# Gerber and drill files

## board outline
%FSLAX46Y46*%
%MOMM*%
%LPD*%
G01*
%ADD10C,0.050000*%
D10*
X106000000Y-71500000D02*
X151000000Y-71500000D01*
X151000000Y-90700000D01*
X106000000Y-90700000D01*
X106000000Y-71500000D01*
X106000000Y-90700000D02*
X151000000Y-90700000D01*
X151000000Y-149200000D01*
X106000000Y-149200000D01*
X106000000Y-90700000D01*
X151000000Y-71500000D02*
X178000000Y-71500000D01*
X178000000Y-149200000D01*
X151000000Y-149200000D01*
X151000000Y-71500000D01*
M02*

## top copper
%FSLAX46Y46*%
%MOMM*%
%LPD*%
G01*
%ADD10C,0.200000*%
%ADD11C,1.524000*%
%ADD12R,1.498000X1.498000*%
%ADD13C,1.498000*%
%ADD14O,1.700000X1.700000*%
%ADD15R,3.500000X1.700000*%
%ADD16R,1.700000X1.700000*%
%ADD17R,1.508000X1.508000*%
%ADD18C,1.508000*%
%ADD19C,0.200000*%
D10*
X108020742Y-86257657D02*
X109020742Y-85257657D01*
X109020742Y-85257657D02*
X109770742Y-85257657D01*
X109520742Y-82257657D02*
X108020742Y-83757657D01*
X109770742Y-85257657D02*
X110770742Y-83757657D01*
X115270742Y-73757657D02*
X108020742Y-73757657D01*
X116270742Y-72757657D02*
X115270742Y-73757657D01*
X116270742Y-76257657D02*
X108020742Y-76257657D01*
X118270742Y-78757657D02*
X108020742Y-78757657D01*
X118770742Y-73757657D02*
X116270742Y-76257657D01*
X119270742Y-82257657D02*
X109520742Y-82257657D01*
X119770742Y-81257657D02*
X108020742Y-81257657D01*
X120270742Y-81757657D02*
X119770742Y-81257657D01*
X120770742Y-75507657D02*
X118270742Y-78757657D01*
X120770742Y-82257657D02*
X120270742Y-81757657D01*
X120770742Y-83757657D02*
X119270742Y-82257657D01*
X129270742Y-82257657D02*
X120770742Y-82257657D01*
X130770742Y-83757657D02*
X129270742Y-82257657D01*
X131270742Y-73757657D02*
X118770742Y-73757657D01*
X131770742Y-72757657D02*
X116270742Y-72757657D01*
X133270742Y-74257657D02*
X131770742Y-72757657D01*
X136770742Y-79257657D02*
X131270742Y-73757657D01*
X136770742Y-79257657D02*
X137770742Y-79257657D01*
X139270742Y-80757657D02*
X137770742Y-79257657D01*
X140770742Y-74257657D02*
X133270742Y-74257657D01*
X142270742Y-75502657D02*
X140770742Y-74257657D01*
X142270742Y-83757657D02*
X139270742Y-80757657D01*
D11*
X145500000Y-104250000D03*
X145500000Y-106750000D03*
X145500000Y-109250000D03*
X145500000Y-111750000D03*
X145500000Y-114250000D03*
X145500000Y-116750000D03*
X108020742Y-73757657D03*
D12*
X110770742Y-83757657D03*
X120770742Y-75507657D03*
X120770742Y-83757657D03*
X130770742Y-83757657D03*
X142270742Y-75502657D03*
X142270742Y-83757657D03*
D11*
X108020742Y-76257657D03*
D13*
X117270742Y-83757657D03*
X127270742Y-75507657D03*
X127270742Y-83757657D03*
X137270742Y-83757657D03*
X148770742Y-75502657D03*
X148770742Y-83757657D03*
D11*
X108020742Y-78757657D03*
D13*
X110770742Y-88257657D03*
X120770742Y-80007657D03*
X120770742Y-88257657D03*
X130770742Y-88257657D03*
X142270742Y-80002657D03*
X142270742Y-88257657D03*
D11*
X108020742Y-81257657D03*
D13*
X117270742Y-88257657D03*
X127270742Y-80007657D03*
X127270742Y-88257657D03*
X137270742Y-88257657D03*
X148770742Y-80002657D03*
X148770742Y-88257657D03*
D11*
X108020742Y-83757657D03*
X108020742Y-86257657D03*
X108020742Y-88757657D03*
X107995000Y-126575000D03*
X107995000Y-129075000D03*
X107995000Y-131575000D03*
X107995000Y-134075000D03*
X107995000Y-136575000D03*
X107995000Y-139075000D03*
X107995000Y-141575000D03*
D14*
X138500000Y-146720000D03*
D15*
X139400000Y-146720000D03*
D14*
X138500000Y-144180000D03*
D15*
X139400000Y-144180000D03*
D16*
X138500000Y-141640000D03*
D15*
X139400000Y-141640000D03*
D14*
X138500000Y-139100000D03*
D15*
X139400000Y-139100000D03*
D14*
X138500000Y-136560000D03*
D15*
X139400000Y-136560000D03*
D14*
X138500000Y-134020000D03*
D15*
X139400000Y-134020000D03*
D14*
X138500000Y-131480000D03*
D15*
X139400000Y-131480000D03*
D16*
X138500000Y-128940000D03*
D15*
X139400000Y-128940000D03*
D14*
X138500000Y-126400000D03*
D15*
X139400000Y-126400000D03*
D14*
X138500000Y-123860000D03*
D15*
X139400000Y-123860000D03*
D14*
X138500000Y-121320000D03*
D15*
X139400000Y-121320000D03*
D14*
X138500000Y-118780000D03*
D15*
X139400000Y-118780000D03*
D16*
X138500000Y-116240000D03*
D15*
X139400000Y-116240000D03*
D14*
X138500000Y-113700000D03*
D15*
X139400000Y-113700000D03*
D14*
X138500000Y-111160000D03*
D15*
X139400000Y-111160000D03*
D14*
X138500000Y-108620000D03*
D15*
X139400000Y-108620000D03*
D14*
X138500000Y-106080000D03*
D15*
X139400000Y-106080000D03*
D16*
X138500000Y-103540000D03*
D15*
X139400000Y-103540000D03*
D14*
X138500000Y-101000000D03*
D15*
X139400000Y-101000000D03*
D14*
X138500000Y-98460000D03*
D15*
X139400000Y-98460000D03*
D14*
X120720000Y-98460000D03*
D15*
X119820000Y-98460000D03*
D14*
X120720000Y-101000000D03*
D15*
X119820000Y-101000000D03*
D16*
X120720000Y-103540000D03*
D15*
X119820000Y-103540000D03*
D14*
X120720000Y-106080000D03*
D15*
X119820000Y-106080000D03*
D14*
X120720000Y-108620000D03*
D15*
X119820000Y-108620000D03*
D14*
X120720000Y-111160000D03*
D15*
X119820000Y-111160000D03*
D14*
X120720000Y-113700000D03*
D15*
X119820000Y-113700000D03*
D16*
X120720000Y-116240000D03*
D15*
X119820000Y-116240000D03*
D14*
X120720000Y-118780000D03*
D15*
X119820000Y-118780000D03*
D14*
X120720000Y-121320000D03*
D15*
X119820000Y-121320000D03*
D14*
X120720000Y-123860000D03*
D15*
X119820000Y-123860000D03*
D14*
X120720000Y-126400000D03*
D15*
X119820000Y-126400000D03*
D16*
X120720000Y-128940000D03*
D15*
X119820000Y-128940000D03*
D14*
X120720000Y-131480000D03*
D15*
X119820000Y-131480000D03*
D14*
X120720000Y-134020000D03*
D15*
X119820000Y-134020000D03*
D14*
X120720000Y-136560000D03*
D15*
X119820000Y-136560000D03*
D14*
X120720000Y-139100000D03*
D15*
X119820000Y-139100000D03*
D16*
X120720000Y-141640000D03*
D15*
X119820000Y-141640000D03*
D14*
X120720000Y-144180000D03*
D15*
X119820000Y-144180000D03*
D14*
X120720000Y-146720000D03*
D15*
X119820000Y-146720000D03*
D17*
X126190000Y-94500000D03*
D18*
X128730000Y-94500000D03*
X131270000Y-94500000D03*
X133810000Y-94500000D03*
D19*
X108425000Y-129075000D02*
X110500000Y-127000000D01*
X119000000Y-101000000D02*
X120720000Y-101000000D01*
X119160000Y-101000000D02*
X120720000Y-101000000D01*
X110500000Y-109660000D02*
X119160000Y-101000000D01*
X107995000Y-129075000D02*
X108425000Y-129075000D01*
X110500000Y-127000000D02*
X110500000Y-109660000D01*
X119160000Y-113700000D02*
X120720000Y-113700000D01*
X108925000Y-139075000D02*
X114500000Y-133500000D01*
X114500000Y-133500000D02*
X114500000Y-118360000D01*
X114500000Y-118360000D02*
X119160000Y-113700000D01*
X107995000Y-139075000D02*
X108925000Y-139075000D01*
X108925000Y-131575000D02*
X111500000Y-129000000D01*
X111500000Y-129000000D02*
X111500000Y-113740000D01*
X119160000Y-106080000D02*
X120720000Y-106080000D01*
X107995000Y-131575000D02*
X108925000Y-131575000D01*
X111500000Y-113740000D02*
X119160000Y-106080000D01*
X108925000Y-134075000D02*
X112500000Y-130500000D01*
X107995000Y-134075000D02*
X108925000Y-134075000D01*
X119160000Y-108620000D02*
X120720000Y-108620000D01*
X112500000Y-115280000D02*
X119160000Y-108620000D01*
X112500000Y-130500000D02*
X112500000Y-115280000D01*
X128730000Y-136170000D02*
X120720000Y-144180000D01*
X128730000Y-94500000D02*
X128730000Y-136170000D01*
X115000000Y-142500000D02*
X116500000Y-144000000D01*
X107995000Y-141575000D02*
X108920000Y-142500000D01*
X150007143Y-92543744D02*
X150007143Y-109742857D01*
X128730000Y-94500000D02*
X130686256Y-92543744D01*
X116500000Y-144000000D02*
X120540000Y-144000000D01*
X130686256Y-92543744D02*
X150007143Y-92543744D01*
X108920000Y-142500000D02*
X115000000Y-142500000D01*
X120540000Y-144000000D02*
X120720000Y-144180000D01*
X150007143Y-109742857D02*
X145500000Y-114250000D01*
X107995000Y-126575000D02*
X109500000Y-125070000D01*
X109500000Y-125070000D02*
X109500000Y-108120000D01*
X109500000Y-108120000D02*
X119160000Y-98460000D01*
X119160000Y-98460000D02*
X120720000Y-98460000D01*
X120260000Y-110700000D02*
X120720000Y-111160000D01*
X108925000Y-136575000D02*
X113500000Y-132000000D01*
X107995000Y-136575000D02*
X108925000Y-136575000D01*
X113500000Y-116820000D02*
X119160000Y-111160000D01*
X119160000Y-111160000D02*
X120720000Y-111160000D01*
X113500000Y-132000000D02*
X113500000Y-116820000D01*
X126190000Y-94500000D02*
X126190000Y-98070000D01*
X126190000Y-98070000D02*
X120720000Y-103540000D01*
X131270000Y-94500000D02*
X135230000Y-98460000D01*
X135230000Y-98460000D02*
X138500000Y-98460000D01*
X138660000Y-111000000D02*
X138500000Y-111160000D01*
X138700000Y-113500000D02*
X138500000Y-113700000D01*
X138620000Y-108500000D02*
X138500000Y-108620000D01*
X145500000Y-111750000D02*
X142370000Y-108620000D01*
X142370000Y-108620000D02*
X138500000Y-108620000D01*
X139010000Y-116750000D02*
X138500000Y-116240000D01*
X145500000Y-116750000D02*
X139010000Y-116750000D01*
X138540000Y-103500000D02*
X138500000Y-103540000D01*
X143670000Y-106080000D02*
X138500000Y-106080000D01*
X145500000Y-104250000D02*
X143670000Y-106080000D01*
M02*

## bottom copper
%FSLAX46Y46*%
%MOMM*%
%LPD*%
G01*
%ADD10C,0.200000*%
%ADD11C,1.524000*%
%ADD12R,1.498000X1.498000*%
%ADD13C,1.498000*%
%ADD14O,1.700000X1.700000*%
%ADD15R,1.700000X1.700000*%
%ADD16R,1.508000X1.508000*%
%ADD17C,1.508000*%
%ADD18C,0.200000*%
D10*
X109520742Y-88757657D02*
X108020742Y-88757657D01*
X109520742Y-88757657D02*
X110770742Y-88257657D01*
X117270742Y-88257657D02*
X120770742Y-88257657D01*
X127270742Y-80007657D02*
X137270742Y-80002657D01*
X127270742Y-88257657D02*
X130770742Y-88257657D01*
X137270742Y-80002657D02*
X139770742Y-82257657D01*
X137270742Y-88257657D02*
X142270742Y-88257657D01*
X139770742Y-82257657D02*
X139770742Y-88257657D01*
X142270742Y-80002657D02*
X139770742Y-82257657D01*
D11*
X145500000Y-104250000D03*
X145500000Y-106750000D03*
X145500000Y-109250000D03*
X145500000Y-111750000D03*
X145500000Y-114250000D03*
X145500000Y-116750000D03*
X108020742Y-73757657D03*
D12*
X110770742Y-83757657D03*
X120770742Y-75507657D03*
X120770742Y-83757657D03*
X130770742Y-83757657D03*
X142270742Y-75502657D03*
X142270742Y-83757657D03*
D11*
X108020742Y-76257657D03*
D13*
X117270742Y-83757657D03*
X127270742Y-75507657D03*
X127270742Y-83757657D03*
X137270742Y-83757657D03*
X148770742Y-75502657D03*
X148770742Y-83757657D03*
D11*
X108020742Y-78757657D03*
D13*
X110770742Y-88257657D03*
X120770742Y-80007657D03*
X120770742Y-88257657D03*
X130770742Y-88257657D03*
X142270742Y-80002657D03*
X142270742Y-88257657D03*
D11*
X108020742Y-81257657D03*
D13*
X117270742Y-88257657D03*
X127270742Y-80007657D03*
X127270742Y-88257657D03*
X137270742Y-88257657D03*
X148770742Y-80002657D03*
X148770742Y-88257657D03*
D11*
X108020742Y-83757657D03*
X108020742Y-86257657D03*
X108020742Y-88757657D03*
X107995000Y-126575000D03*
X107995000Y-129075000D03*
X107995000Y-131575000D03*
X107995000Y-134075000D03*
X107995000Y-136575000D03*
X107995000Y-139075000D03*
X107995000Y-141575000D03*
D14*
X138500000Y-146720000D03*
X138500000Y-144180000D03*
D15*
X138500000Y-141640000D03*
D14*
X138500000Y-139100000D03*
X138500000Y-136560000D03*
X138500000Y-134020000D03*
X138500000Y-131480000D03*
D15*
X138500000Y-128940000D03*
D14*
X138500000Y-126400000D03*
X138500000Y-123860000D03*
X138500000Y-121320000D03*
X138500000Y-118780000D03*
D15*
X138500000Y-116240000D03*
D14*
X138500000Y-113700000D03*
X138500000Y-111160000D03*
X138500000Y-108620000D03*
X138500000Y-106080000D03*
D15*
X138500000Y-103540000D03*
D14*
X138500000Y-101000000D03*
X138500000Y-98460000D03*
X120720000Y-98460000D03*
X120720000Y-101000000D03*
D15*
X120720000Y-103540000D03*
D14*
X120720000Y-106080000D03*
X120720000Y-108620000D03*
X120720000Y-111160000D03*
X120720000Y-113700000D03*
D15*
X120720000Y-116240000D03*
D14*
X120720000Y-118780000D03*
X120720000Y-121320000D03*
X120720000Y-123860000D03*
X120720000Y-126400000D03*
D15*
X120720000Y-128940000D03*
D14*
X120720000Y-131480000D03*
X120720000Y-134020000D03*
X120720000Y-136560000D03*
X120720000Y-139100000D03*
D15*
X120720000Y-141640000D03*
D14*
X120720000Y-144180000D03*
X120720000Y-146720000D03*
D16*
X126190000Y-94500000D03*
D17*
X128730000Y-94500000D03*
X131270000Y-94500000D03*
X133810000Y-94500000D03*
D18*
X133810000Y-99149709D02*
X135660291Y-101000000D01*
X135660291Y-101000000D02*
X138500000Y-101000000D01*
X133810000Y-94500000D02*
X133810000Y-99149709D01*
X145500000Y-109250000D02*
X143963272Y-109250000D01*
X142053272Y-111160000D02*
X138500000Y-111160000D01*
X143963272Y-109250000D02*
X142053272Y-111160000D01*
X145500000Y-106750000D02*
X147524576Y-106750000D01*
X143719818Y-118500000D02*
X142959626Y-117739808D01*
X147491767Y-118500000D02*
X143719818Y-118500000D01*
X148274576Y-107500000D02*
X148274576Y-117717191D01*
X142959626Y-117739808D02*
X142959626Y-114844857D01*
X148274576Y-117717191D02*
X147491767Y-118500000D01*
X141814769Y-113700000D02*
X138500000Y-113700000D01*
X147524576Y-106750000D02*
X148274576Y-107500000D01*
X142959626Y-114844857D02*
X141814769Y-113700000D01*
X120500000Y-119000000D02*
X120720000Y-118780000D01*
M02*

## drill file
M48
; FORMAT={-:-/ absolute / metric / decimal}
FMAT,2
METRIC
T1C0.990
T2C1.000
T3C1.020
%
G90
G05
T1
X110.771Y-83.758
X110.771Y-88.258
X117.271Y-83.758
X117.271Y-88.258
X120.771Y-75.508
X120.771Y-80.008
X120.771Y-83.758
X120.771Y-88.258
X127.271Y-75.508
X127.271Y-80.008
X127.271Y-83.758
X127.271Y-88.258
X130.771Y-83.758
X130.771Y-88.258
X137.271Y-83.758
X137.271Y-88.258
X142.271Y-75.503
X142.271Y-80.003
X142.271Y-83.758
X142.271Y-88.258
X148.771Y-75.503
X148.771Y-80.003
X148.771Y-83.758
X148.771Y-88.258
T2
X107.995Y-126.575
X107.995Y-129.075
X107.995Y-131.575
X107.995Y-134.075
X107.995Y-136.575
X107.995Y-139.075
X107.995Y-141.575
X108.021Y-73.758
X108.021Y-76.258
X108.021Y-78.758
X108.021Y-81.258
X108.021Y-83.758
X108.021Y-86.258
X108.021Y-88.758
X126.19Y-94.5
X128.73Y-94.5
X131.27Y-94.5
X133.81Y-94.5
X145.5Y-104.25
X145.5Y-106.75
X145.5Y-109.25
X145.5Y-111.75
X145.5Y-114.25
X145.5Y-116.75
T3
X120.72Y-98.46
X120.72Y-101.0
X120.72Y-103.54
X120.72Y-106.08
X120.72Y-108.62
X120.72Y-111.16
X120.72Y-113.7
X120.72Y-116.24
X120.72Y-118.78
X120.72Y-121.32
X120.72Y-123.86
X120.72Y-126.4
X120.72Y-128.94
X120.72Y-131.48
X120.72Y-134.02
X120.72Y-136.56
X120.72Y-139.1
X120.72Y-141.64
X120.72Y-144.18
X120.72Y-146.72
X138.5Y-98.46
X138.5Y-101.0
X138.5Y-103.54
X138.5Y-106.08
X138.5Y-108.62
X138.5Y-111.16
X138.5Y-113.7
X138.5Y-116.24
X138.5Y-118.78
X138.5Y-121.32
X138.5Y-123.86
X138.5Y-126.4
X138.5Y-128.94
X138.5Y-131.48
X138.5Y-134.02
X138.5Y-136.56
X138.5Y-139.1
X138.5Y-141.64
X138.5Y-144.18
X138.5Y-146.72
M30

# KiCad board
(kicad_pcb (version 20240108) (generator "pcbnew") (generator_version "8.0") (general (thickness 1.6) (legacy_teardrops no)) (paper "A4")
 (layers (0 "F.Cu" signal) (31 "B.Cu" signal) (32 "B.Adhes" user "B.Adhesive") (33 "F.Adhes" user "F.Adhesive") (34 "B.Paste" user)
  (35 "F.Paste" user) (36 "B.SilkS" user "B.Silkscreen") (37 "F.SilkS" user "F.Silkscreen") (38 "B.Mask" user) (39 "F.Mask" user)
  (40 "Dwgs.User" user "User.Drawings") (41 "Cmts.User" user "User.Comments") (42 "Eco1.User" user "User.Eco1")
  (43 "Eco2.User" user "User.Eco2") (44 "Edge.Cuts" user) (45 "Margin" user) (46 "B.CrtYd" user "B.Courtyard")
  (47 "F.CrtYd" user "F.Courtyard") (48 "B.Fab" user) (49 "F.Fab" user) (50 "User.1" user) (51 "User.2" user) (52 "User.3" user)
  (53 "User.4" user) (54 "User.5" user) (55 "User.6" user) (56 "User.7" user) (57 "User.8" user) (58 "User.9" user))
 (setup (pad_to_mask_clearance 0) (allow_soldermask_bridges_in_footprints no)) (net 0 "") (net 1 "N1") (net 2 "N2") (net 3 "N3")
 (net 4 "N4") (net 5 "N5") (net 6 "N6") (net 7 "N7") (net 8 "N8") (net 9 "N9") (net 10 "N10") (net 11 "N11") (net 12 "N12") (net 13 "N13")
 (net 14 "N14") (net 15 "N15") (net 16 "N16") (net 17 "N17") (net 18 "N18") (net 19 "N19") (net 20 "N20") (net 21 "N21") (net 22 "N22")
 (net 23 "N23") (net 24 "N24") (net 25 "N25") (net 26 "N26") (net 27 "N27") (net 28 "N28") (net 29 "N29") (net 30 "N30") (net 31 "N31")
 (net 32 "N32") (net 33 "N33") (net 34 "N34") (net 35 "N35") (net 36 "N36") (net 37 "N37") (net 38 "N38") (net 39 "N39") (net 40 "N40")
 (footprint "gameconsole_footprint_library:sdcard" (layer "F.Cu") (at 148.75 98.5 -90)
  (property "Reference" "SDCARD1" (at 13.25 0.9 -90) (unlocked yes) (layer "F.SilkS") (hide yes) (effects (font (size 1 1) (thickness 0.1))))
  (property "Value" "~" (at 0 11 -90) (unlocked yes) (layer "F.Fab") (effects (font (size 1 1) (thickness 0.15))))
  (pad "1" thru_hole circle (at 5.75 3.25 270) (size 1.524 1.524) (drill 1) (layers "*.Cu" "*.Mask") (remove_unused_layers no) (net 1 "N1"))
  (pad "2" thru_hole circle (at 8.25 3.25 270) (size 1.524 1.524) (drill 1) (layers "*.Cu" "*.Mask") (remove_unused_layers no) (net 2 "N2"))
  (pad "3" thru_hole circle (at 10.75 3.25 270) (size 1.524 1.524) (drill 1) (layers "*.Cu" "*.Mask") (remove_unused_layers no) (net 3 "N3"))
  (pad "4" thru_hole circle (at 13.25 3.25 270) (size 1.524 1.524) (drill 1) (layers "*.Cu" "*.Mask") (remove_unused_layers no) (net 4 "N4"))
  (pad "5" thru_hole circle (at 15.75 3.25 270) (size 1.524 1.524) (drill 1) (layers "*.Cu" "*.Mask") (remove_unused_layers no) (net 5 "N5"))
  (pad "6" thru_hole circle (at 18.25 3.25 270) (size 1.524 1.524) (drill 1) (layers "*.Cu" "*.Mask") (remove_unused_layers no) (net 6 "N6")))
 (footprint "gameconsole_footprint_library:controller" (layer "F.Cu") (at 106.525742 72.257657)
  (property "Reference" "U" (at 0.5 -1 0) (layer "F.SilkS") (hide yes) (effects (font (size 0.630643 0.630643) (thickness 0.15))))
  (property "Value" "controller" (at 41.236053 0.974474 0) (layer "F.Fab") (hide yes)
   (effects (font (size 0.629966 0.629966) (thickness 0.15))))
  (fp_line (start 1.495 14) (end 2.495 13) (stroke (width 0.2) (type default)) (layer "F.Cu"))
  (fp_line (start 2.495 13) (end 3.245 13) (stroke (width 0.2) (type default)) (layer "F.Cu"))
  (fp_line (start 2.995 10) (end 1.495 11.5) (stroke (width 0.2) (type default)) (layer "F.Cu"))
  (fp_line (start 3.245 13) (end 4.245 11.5) (stroke (width 0.2) (type default)) (layer "F.Cu"))
  (fp_line (start 8.745 1.5) (end 1.495 1.5) (stroke (width 0.2) (type default)) (layer "F.Cu"))
  (fp_line (start 9.745 0.5) (end 8.745 1.5) (stroke (width 0.2) (type default)) (layer "F.Cu"))
  (fp_line (start 9.745 4) (end 1.495 4) (stroke (width 0.2) (type default)) (layer "F.Cu"))
  (fp_line (start 11.745 6.5) (end 1.495 6.5) (stroke (width 0.2) (type default)) (layer "F.Cu"))
  (fp_line (start 12.245 1.5) (end 9.745 4) (stroke (width 0.2) (type default)) (layer "F.Cu"))
  (fp_line (start 12.745 10) (end 2.995 10) (stroke (width 0.2) (type default)) (layer "F.Cu"))
  (fp_line (start 13.245 9) (end 1.495 9) (stroke (width 0.2) (type default)) (layer "F.Cu"))
  (fp_line (start 13.745 9.5) (end 13.245 9) (stroke (width 0.2) (type default)) (layer "F.Cu"))
  (fp_line (start 14.245 3.25) (end 11.745 6.5) (stroke (width 0.2) (type default)) (layer "F.Cu"))
  (fp_line (start 14.245 10) (end 13.745 9.5) (stroke (width 0.2) (type default)) (layer "F.Cu"))
  (fp_line (start 14.245 11.5) (end 12.745 10) (stroke (width 0.2) (type default)) (layer "F.Cu"))
  (fp_line (start 22.745 10) (end 14.245 10) (stroke (width 0.2) (type default)) (layer "F.Cu"))
  (fp_line (start 24.245 11.5) (end 22.745 10) (stroke (width 0.2) (type default)) (layer "F.Cu"))
  (fp_line (start 24.745 1.5) (end 12.245 1.5) (stroke (width 0.2) (type default)) (layer "F.Cu"))
  (fp_line (start 25.245 0.5) (end 9.745 0.5) (stroke (width 0.2) (type default)) (layer "F.Cu"))
  (fp_line (start 26.745 2) (end 25.245 0.5) (stroke (width 0.2) (type default)) (layer "F.Cu"))
  (fp_line (start 30.245 7) (end 24.745 1.5) (stroke (width 0.2) (type default)) (layer "F.Cu"))
  (fp_line (start 30.245 7) (end 31.245 7) (stroke (width 0.2) (type default)) (layer "F.Cu"))
  (fp_line (start 32.745 8.5) (end 31.245 7) (stroke (width 0.2) (type default)) (layer "F.Cu"))
  (fp_line (start 34.245 2) (end 26.745 2) (stroke (width 0.2) (type default)) (layer "F.Cu"))
  (fp_line (start 35.745 3.245) (end 34.245 2) (stroke (width 0.2) (type default)) (layer "F.Cu"))
  (fp_line (start 35.745 11.5) (end 32.745 8.5) (stroke (width 0.2) (type default)) (layer "F.Cu"))
  (fp_line (start 2.995 16.5) (end 1.495 16.5) (stroke (width 0.2) (type default)) (layer "B.Cu"))
  (fp_line (start 2.995 16.5) (end 4.245 16) (stroke (width 0.2) (type default)) (layer "B.Cu"))
  (fp_line (start 10.745 16) (end 14.245 16) (stroke (width 0.2) (type default)) (layer "B.Cu"))
  (fp_line (start 20.745 7.75) (end 30.745 7.745) (stroke (width 0.2) (type default)) (layer "B.Cu"))
  (fp_line (start 20.745 16) (end 24.245 16) (stroke (width 0.2) (type default)) (layer "B.Cu"))
  (fp_line (start 30.745 7.745) (end 33.245 10) (stroke (width 0.2) (type default)) (layer "B.Cu"))
  (fp_line (start 30.745 16) (end 35.745 16) (stroke (width 0.2) (type default)) (layer "B.Cu"))
  (fp_line (start 33.245 10) (end 33.245 16) (stroke (width 0.2) (type default)) (layer "B.Cu"))
  (fp_line (start 35.745 7.745) (end 33.245 10) (stroke (width 0.2) (type default)) (layer "B.Cu"))
  (pad "1" thru_hole circle (at 1.495 1.5) (size 1.524 1.524) (drill 1) (layers "*.Cu" "*.Mask") (remove_unused_layers no))
  (pad "1" thru_hole rect (at 4.245 11.5) (size 1.498 1.498) (drill 0.99) (layers "*.Cu" "*.Mask") (remove_unused_layers no)
   (solder_mask_margin 0.102))
  (pad "1" thru_hole rect (at 14.245 3.25) (size 1.498 1.498) (drill 0.99) (layers "*.Cu" "*.Mask") (remove_unused_layers no)
   (solder_mask_margin 0.102))
  (pad "1" thru_hole rect (at 14.245 11.5) (size 1.498 1.498) (drill 0.99) (layers "*.Cu" "*.Mask") (remove_unused_layers no)
   (solder_mask_margin 0.102))
  (pad "1" thru_hole rect (at 24.245 11.5) (size 1.498 1.498) (drill 0.99) (layers "*.Cu" "*.Mask") (remove_unused_layers no)
   (solder_mask_margin 0.102))
  (pad "1" thru_hole rect (at 35.745 3.245) (size 1.498 1.498) (drill 0.99) (layers "*.Cu" "*.Mask") (remove_unused_layers no)
   (solder_mask_margin 0.102))
  (pad "1" thru_hole rect (at 35.745 11.5) (size 1.498 1.498) (drill 0.99) (layers "*.Cu" "*.Mask") (remove_unused_layers no)
   (solder_mask_margin 0.102))
  (pad "2" thru_hole circle (at 1.495 4) (size 1.524 1.524) (drill 1) (layers "*.Cu" "*.Mask") (remove_unused_layers no))
  (pad "2" thru_hole circle (at 10.745 11.5) (size 1.498 1.498) (drill 0.99) (layers "*.Cu" "*.Mask") (remove_unused_layers no)
   (solder_mask_margin 0.102))
  (pad "2" thru_hole circle (at 20.745 3.25) (size 1.498 1.498) (drill 0.99) (layers "*.Cu" "*.Mask") (remove_unused_layers no)
   (solder_mask_margin 0.102))
  (pad "2" thru_hole circle (at 20.745 11.5) (size 1.498 1.498) (drill 0.99) (layers "*.Cu" "*.Mask") (remove_unused_layers no)
   (solder_mask_margin 0.102))
  (pad "2" thru_hole circle (at 30.745 11.5) (size 1.498 1.498) (drill 0.99) (layers "*.Cu" "*.Mask") (remove_unused_layers no)
   (solder_mask_margin 0.102))
  (pad "2" thru_hole circle (at 42.245 3.245) (size 1.498 1.498) (drill 0.99) (layers "*.Cu" "*.Mask") (remove_unused_layers no)
   (solder_mask_margin 0.102))
  (pad "2" thru_hole circle (at 42.245 11.5) (size 1.498 1.498) (drill 0.99) (layers "*.Cu" "*.Mask") (remove_unused_layers no)
   (solder_mask_margin 0.102))
  (pad "3" thru_hole circle (at 1.495 6.5) (size 1.524 1.524) (drill 1) (layers "*.Cu" "*.Mask") (remove_unused_layers no))
  (pad "3" thru_hole circle (at 4.245 16) (size 1.498 1.498) (drill 0.99) (layers "*.Cu" "*.Mask") (remove_unused_layers no)
   (solder_mask_margin 0.102))
  (pad "3" thru_hole circle (at 14.245 7.75) (size 1.498 1.498) (drill 0.99) (layers "*.Cu" "*.Mask") (remove_unused_layers no)
   (solder_mask_margin 0.102))
  (pad "3" thru_hole circle (at 14.245 16) (size 1.498 1.498) (drill 0.99) (layers "*.Cu" "*.Mask") (remove_unused_layers no)
   (solder_mask_margin 0.102))
  (pad "3" thru_hole circle (at 24.245 16) (size 1.498 1.498) (drill 0.99) (layers "*.Cu" "*.Mask") (remove_unused_layers no)
   (solder_mask_margin 0.102))
  (pad "3" thru_hole circle (at 35.745 7.745) (size 1.498 1.498) (drill 0.99) (layers "*.Cu" "*.Mask") (remove_unused_layers no)
   (solder_mask_margin 0.102))
  (pad "3" thru_hole circle (at 35.745 16) (size 1.498 1.498) (drill 0.99) (layers "*.Cu" "*.Mask") (remove_unused_layers no)
   (solder_mask_margin 0.102))
  (pad "4" thru_hole circle (at 1.495 9) (size 1.524 1.524) (drill 1) (layers "*.Cu" "*.Mask") (remove_unused_layers no))
  (pad "4" thru_hole circle (at 10.745 16) (size 1.498 1.498) (drill 0.99) (layers "*.Cu" "*.Mask") (remove_unused_layers no)
   (solder_mask_margin 0.102))
  (pad "4" thru_hole circle (at 20.745 7.75) (size 1.498 1.498) (drill 0.99) (layers "*.Cu" "*.Mask") (remove_unused_layers no)
   (solder_mask_margin 0.102))
  (pad "4" thru_hole circle (at 20.745 16) (size 1.498 1.498) (drill 0.99) (layers "*.Cu" "*.Mask") (remove_unused_layers no)
   (solder_mask_margin 0.102))
  (pad "4" thru_hole circle (at 30.745 16) (size 1.498 1.498) (drill 0.99) (layers "*.Cu" "*.Mask") (remove_unused_layers no)
   (solder_mask_margin 0.102))
  (pad "4" thru_hole circle (at 42.245 7.745) (size 1.498 1.498) (drill 0.99) (layers "*.Cu" "*.Mask") (remove_unused_layers no)
   (solder_mask_margin 0.102))
  (pad "4" thru_hole circle (at 42.245 16) (size 1.498 1.498) (drill 0.99) (layers "*.Cu" "*.Mask") (remove_unused_layers no)
   (solder_mask_margin 0.102))
  (pad "5" thru_hole circle (at 1.495 11.5) (size 1.524 1.524) (drill 1) (layers "*.Cu" "*.Mask") (remove_unused_layers no))
  (pad "6" thru_hole circle (at 1.495 14) (size 1.524 1.524) (drill 1) (layers "*.Cu" "*.Mask") (remove_unused_layers no))
  (pad "7" thru_hole circle (at 1.495 16.5) (size 1.524 1.524) (drill 1) (layers "*.Cu" "*.Mask") (remove_unused_layers no)))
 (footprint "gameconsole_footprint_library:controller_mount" (layer "F.Cu") (at 106.5 125.075)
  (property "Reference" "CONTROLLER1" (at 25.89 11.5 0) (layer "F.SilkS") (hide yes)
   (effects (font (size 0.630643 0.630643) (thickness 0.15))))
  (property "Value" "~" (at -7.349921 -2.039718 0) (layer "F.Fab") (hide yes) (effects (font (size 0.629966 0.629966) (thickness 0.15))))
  (pad "1" thru_hole circle (at 1.495 1.5) (size 1.524 1.524) (drill 1) (layers "*.Cu" "*.Mask") (remove_unused_layers no) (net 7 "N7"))
  (pad "2" thru_hole circle (at 1.495 4) (size 1.524 1.524) (drill 1) (layers "*.Cu" "*.Mask") (remove_unused_layers no) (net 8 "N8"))
  (pad "3" thru_hole circle (at 1.495 6.5) (size 1.524 1.524) (drill 1) (layers "*.Cu" "*.Mask") (remove_unused_layers no) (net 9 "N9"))
  (pad "4" thru_hole circle (at 1.495 9) (size 1.524 1.524) (drill 1) (layers "*.Cu" "*.Mask") (remove_unused_layers no) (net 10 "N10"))
  (pad "5" thru_hole circle (at 1.495 11.5) (size 1.524 1.524) (drill 1) (layers "*.Cu" "*.Mask") (remove_unused_layers no) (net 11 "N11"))
  (pad "6" thru_hole circle (at 1.495 14) (size 1.524 1.524) (drill 1) (layers "*.Cu" "*.Mask") (remove_unused_layers no) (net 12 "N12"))
  (pad "7" thru_hole circle (at 1.495 16.5) (size 1.524 1.524) (drill 1) (layers "*.Cu" "*.Mask") (remove_unused_layers no) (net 5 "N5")))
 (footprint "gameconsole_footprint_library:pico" (layer "F.Cu") (at 129.61 122.59 180)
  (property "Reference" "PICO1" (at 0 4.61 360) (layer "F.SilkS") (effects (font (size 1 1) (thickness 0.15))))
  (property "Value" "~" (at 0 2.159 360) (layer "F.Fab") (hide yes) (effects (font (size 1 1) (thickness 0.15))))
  (pad "1" thru_hole oval (at -8.89 -24.13 180) (size 1.7 1.7) (drill 1.02) (layers "*.Cu" "*.Mask") (remove_unused_layers no)
   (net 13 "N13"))
  (pad "1" smd rect (at -8.89 -24.13 180) (size 3.5 1.7) (drill (offset -0.9 0)) (layers "F.Cu" "F.Mask") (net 13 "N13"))
  (pad "2" thru_hole oval (at -8.89 -21.59 180) (size 1.7 1.7) (drill 1.02) (layers "*.Cu" "*.Mask") (remove_unused_layers no)
   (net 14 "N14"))
  (pad "2" smd rect (at -8.89 -21.59 180) (size 3.5 1.7) (drill (offset -0.9 0)) (layers "F.Cu" "F.Mask") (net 14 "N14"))
  (pad "3" thru_hole rect (at -8.89 -19.05 180) (size 1.7 1.7) (drill 1.02) (layers "*.Cu" "*.Mask") (remove_unused_layers no)
   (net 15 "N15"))
  (pad "3" smd rect (at -8.89 -19.05 180) (size 3.5 1.7) (drill (offset -0.9 0)) (layers "F.Cu" "F.Mask") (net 15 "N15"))
  (pad "4" thru_hole oval (at -8.89 -16.51 180) (size 1.7 1.7) (drill 1.02) (layers "*.Cu" "*.Mask") (remove_unused_layers no)
   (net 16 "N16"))
  (pad "4" smd rect (at -8.89 -16.51 180) (size 3.5 1.7) (drill (offset -0.9 0)) (layers "F.Cu" "F.Mask") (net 16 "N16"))
  (pad "5" thru_hole oval (at -8.89 -13.97 180) (size 1.7 1.7) (drill 1.02) (layers "*.Cu" "*.Mask") (remove_unused_layers no)
   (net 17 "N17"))
  (pad "5" smd rect (at -8.89 -13.97 180) (size 3.5 1.7) (drill (offset -0.9 0)) (layers "F.Cu" "F.Mask") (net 17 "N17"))
  (pad "6" thru_hole oval (at -8.89 -11.43 180) (size 1.7 1.7) (drill 1.02) (layers "*.Cu" "*.Mask") (remove_unused_layers no)
   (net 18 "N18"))
  (pad "6" smd rect (at -8.89 -11.43 180) (size 3.5 1.7) (drill (offset -0.9 0)) (layers "F.Cu" "F.Mask") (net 18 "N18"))
  (pad "7" thru_hole oval (at -8.89 -8.89 180) (size 1.7 1.7) (drill 1.02) (layers "*.Cu" "*.Mask") (remove_unused_layers no) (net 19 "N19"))
  (pad "7" smd rect (at -8.89 -8.89 180) (size 3.5 1.7) (drill (offset -0.9 0)) (layers "F.Cu" "F.Mask") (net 19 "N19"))
  (pad "8" thru_hole rect (at -8.89 -6.35 180) (size 1.7 1.7) (drill 1.02) (layers "*.Cu" "*.Mask") (remove_unused_layers no) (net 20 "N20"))
  (pad "8" smd rect (at -8.89 -6.35 180) (size 3.5 1.7) (drill (offset -0.9 0)) (layers "F.Cu" "F.Mask") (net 20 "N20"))
  (pad "9" thru_hole oval (at -8.89 -3.81 180) (size 1.7 1.7) (drill 1.02) (layers "*.Cu" "*.Mask") (remove_unused_layers no) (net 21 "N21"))
  (pad "9" smd rect (at -8.89 -3.81 180) (size 3.5 1.7) (drill (offset -0.9 0)) (layers "F.Cu" "F.Mask") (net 21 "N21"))
  (pad "10" thru_hole oval (at -8.89 -1.27 180) (size 1.7 1.7) (drill 1.02) (layers "*.Cu" "*.Mask") (remove_unused_layers no)
   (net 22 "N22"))
  (pad "10" smd rect (at -8.89 -1.27 180) (size 3.5 1.7) (drill (offset -0.9 0)) (layers "F.Cu" "F.Mask") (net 22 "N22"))
  (pad "11" thru_hole oval (at -8.89 1.27 180) (size 1.7 1.7) (drill 1.02) (layers "*.Cu" "*.Mask") (remove_unused_layers no) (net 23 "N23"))
  (pad "11" smd rect (at -8.89 1.27 180) (size 3.5 1.7) (drill (offset -0.9 0)) (layers "F.Cu" "F.Mask") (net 23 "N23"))
  (pad "12" thru_hole oval (at -8.89 3.81 180) (size 1.7 1.7) (drill 1.02) (layers "*.Cu" "*.Mask") (remove_unused_layers no) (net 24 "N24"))
  (pad "12" smd rect (at -8.89 3.81 180) (size 3.5 1.7) (drill (offset -0.9 0)) (layers "F.Cu" "F.Mask") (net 24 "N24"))
  (pad "13" thru_hole rect (at -8.89 6.35 180) (size 1.7 1.7) (drill 1.02) (layers "*.Cu" "*.Mask") (remove_unused_layers no) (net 6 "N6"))
  (pad "13" smd rect (at -8.89 6.35 180) (size 3.5 1.7) (drill (offset -0.9 0)) (layers "F.Cu" "F.Mask") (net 6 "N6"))
  (pad "14" thru_hole oval (at -8.89 8.89 180) (size 1.7 1.7) (drill 1.02) (layers "*.Cu" "*.Mask") (remove_unused_layers no) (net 2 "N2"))
  (pad "14" smd rect (at -8.89 8.89 180) (size 3.5 1.7) (drill (offset -0.9 0)) (layers "F.Cu" "F.Mask") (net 2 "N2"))
  (pad "15" thru_hole oval (at -8.89 11.43 180) (size 1.7 1.7) (drill 1.02) (layers "*.Cu" "*.Mask") (remove_unused_layers no) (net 3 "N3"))
  (pad "15" smd rect (at -8.89 11.43 180) (size 3.5 1.7) (drill (offset -0.9 0)) (layers "F.Cu" "F.Mask") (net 3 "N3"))
  (pad "16" thru_hole oval (at -8.89 13.97 180) (size 1.7 1.7) (drill 1.02) (layers "*.Cu" "*.Mask") (remove_unused_layers no) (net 4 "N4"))
  (pad "16" smd rect (at -8.89 13.97 180) (size 3.5 1.7) (drill (offset -0.9 0)) (layers "F.Cu" "F.Mask") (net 4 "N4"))
  (pad "17" thru_hole oval (at -8.89 16.51 180) (size 1.7 1.7) (drill 1.02) (layers "*.Cu" "*.Mask") (remove_unused_layers no) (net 1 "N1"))
  (pad "17" smd rect (at -8.89 16.51 180) (size 3.5 1.7) (drill (offset -0.9 0)) (layers "F.Cu" "F.Mask") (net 1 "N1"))
  (pad "18" thru_hole rect (at -8.89 19.05 180) (size 1.7 1.7) (drill 1.02) (layers "*.Cu" "*.Mask") (remove_unused_layers no)
   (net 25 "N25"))
  (pad "18" smd rect (at -8.89 19.05 180) (size 3.5 1.7) (drill (offset -0.9 0)) (layers "F.Cu" "F.Mask") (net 25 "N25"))
  (pad "19" thru_hole oval (at -8.89 21.59 180) (size 1.7 1.7) (drill 1.02) (layers "*.Cu" "*.Mask") (remove_unused_layers no)
   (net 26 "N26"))
  (pad "19" smd rect (at -8.89 21.59 180) (size 3.5 1.7) (drill (offset -0.9 0)) (layers "F.Cu" "F.Mask") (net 26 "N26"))
  (pad "20" thru_hole oval (at -8.89 24.13 180) (size 1.7 1.7) (drill 1.02) (layers "*.Cu" "*.Mask") (remove_unused_layers no)
   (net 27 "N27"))
  (pad "20" smd rect (at -8.89 24.13 180) (size 3.5 1.7) (drill (offset -0.9 0)) (layers "F.Cu" "F.Mask") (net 27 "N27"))
  (pad "21" thru_hole oval (at 8.89 24.13 180) (size 1.7 1.7) (drill 1.02) (layers "*.Cu" "*.Mask") (remove_unused_layers no) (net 7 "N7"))
  (pad "21" smd rect (at 8.89 24.13 180) (size 3.5 1.7) (drill (offset 0.9 0)) (layers "F.Cu" "F.Mask") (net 7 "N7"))
  (pad "22" thru_hole oval (at 8.89 21.59 180) (size 1.7 1.7) (drill 1.02) (layers "*.Cu" "*.Mask") (remove_unused_layers no) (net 8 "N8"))
  (pad "22" smd rect (at 8.89 21.59 180) (size 3.5 1.7) (drill (offset 0.9 0)) (layers "F.Cu" "F.Mask") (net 8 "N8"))
  (pad "23" thru_hole rect (at 8.89 19.05 180) (size 1.7 1.7) (drill 1.02) (layers "*.Cu" "*.Mask") (remove_unused_layers no) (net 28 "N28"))
  (pad "23" smd rect (at 8.89 19.05 180) (size 3.5 1.7) (drill (offset 0.9 0)) (layers "F.Cu" "F.Mask") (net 28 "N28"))
  (pad "24" thru_hole oval (at 8.89 16.51 180) (size 1.7 1.7) (drill 1.02) (layers "*.Cu" "*.Mask") (remove_unused_layers no) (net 9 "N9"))
  (pad "24" smd rect (at 8.89 16.51 180) (size 3.5 1.7) (drill (offset 0.9 0)) (layers "F.Cu" "F.Mask") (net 9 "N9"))
  (pad "25" thru_hole oval (at 8.89 13.97 180) (size 1.7 1.7) (drill 1.02) (layers "*.Cu" "*.Mask") (remove_unused_layers no) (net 10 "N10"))
  (pad "25" smd rect (at 8.89 13.97 180) (size 3.5 1.7) (drill (offset 0.9 0)) (layers "F.Cu" "F.Mask") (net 10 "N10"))
  (pad "26" thru_hole oval (at 8.89 11.43 180) (size 1.7 1.7) (drill 1.02) (layers "*.Cu" "*.Mask") (remove_unused_layers no) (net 11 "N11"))
  (pad "26" smd rect (at 8.89 11.43 180) (size 3.5 1.7) (drill (offset 0.9 0)) (layers "F.Cu" "F.Mask") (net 11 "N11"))
  (pad "27" thru_hole oval (at 8.89 8.89 180) (size 1.7 1.7) (drill 1.02) (layers "*.Cu" "*.Mask") (remove_unused_layers no) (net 12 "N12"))
  (pad "27" smd rect (at 8.89 8.89 180) (size 3.5 1.7) (drill (offset 0.9 0)) (layers "F.Cu" "F.Mask") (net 12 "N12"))
  (pad "28" thru_hole rect (at 8.89 6.35 180) (size 1.7 1.7) (drill 1.02) (layers "*.Cu" "*.Mask") (remove_unused_layers no) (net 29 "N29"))
  (pad "28" smd rect (at 8.89 6.35 180) (size 3.5 1.7) (drill (offset 0.9 0)) (layers "F.Cu" "F.Mask") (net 29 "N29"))
  (pad "29" thru_hole oval (at 8.89 3.81 180) (size 1.7 1.7) (drill 1.02) (layers "*.Cu" "*.Mask") (remove_unused_layers no) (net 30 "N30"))
  (pad "29" smd rect (at 8.89 3.81 180) (size 3.5 1.7) (drill (offset 0.9 0)) (layers "F.Cu" "F.Mask") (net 30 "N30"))
  (pad "30" thru_hole oval (at 8.89 1.27 180) (size 1.7 1.7) (drill 1.02) (layers "*.Cu" "*.Mask") (remove_unused_layers no) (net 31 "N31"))
  (pad "30" smd rect (at 8.89 1.27 180) (size 3.5 1.7) (drill (offset 0.9 0)) (layers "F.Cu" "F.Mask") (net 31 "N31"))
  (pad "31" thru_hole oval (at 8.89 -1.27 180) (size 1.7 1.7) (drill 1.02) (layers "*.Cu" "*.Mask") (remove_unused_layers no) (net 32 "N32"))
  (pad "31" smd rect (at 8.89 -1.27 180) (size 3.5 1.7) (drill (offset 0.9 0)) (layers "F.Cu" "F.Mask") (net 32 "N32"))
  (pad "32" thru_hole oval (at 8.89 -3.81 180) (size 1.7 1.7) (drill 1.02) (layers "*.Cu" "*.Mask") (remove_unused_layers no) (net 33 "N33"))
  (pad "32" smd rect (at 8.89 -3.81 180) (size 3.5 1.7) (drill (offset 0.9 0)) (layers "F.Cu" "F.Mask") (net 33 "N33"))
  (pad "33" thru_hole rect (at 8.89 -6.35 180) (size 1.7 1.7) (drill 1.02) (layers "*.Cu" "*.Mask") (remove_unused_layers no) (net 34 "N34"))
  (pad "33" smd rect (at 8.89 -6.35 180) (size 3.5 1.7) (drill (offset 0.9 0)) (layers "F.Cu" "F.Mask") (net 34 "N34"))
  (pad "34" thru_hole oval (at 8.89 -8.89 180) (size 1.7 1.7) (drill 1.02) (layers "*.Cu" "*.Mask") (remove_unused_layers no) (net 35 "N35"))
  (pad "34" smd rect (at 8.89 -8.89 180) (size 3.5 1.7) (drill (offset 0.9 0)) (layers "F.Cu" "F.Mask") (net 35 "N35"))
  (pad "35" thru_hole oval (at 8.89 -11.43 180) (size 1.7 1.7) (drill 1.02) (layers "*.Cu" "*.Mask") (remove_unused_layers no)
   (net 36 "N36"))
  (pad "35" smd rect (at 8.89 -11.43 180) (size 3.5 1.7) (drill (offset 0.9 0)) (layers "F.Cu" "F.Mask") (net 36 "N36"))
  (pad "36" thru_hole oval (at 8.89 -13.97 180) (size 1.7 1.7) (drill 1.02) (layers "*.Cu" "*.Mask") (remove_unused_layers no)
   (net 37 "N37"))
  (pad "36" smd rect (at 8.89 -13.97 180) (size 3.5 1.7) (drill (offset 0.9 0)) (layers "F.Cu" "F.Mask") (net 37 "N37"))
  (pad "37" thru_hole oval (at 8.89 -16.51 180) (size 1.7 1.7) (drill 1.02) (layers "*.Cu" "*.Mask") (remove_unused_layers no)
   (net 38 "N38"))
  (pad "37" smd rect (at 8.89 -16.51 180) (size 3.5 1.7) (drill (offset 0.9 0)) (layers "F.Cu" "F.Mask") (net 38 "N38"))
  (pad "38" thru_hole rect (at 8.89 -19.05 180) (size 1.7 1.7) (drill 1.02) (layers "*.Cu" "*.Mask") (remove_unused_layers no)
   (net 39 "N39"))
  (pad "38" smd rect (at 8.89 -19.05 180) (size 3.5 1.7) (drill (offset 0.9 0)) (layers "F.Cu" "F.Mask") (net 39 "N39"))
  (pad "39" thru_hole oval (at 8.89 -21.59 180) (size 1.7 1.7) (drill 1.02) (layers "*.Cu" "*.Mask") (remove_unused_layers no) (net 5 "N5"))
  (pad "39" smd rect (at 8.89 -21.59 180) (size 3.5 1.7) (drill (offset 0.9 0)) (layers "F.Cu" "F.Mask") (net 5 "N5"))
  (pad "40" thru_hole oval (at 8.89 -24.13 180) (size 1.7 1.7) (drill 1.02) (layers "*.Cu" "*.Mask") (remove_unused_layers no)
   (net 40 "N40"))
  (pad "40" smd rect (at 8.89 -24.13 180) (size 3.5 1.7) (drill (offset 0.9 0)) (layers "F.Cu" "F.Mask") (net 40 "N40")))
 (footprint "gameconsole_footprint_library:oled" (layer "F.Cu") (at 130 106)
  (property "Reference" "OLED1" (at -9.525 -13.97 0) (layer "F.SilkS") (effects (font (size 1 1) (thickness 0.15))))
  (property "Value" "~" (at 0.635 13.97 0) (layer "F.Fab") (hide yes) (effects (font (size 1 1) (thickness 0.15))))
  (pad "1" thru_hole rect (at -3.81 -11.5) (size 1.508 1.508) (drill 1) (layers "*.Cu" "*.Mask") (remove_unused_layers no) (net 28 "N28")
   (solder_mask_margin 0.102))
  (pad "2" thru_hole circle (at -1.27 -11.5) (size 1.508 1.508) (drill 1) (layers "*.Cu" "*.Mask") (remove_unused_layers no) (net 5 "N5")
   (solder_mask_margin 0.102))
  (pad "3" thru_hole circle (at 1.27 -11.5) (size 1.508 1.508) (drill 1) (layers "*.Cu" "*.Mask") (remove_unused_layers no) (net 27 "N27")
   (solder_mask_margin 0.102))
  (pad "4" thru_hole circle (at 3.81 -11.5) (size 1.508 1.508) (drill 1) (layers "*.Cu" "*.Mask") (remove_unused_layers no) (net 26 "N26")
   (solder_mask_margin 0.102)))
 (gr_rect (start 106 71.5) (end 151 90.7) (stroke (width 0.05) (type default)) (fill none) (layer "Edge.Cuts"))
 (gr_rect (start 106 90.7) (end 151 149.2) (stroke (width 0.05) (type default)) (fill none) (layer "Edge.Cuts"))
 (gr_rect (start 151 71.5) (end 178 149.2) (stroke (width 0.05) (type default)) (fill none) (layer "Edge.Cuts"))
 (segment (start 108.425 129.075) (end 110.5 127) (width 0.2) (layer "F.Cu") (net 8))
 (segment (start 119 101) (end 120.72 101) (width 0.2) (layer "F.Cu") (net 8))
 (segment (start 119.16 101) (end 120.72 101) (width 0.2) (layer "F.Cu") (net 8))
 (segment (start 110.5 109.66) (end 119.16 101) (width 0.2) (layer "F.Cu") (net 8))
 (segment (start 107.995 129.075) (end 108.425 129.075) (width 0.2) (layer "F.Cu") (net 8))
 (segment (start 110.5 127) (end 110.5 109.66) (width 0.2) (layer "F.Cu") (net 8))
 (segment (start 119.16 113.7) (end 120.72 113.7) (width 0.2) (layer "F.Cu") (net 12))
 (segment (start 108.925 139.075) (end 114.5 133.5) (width 0.2) (layer "F.Cu") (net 12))
 (segment (start 114.5 133.5) (end 114.5 118.36) (width 0.2) (layer "F.Cu") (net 12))
 (segment (start 114.5 118.36) (end 119.16 113.7) (width 0.2) (layer "F.Cu") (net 12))
 (segment (start 107.995 139.075) (end 108.925 139.075) (width 0.2) (layer "F.Cu") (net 12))
 (segment (start 108.925 131.575) (end 111.5 129) (width 0.2) (layer "F.Cu") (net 9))
 (segment (start 111.5 129) (end 111.5 113.74) (width 0.2) (layer "F.Cu") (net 9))
 (segment (start 119.16 106.08) (end 120.72 106.08) (width 0.2) (layer "F.Cu") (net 9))
 (segment (start 107.995 131.575) (end 108.925 131.575) (width 0.2) (layer "F.Cu") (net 9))
 (segment (start 111.5 113.74) (end 119.16 106.08) (width 0.2) (layer "F.Cu") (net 9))
 (segment (start 108.925 134.075) (end 112.5 130.5) (width 0.2) (layer "F.Cu") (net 10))
 (segment (start 107.995 134.075) (end 108.925 134.075) (width 0.2) (layer "F.Cu") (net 10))
 (segment (start 119.16 108.62) (end 120.72 108.62) (width 0.2) (layer "F.Cu") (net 10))
 (segment (start 112.5 115.28) (end 119.16 108.62) (width 0.2) (layer "F.Cu") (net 10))
 (segment (start 112.5 130.5) (end 112.5 115.28) (width 0.2) (layer "F.Cu") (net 10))
 (segment (start 128.73 136.17) (end 120.72 144.18) (width 0.2) (layer "F.Cu") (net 5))
 (segment (start 128.73 94.5) (end 128.73 136.17) (width 0.2) (layer "F.Cu") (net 5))
 (segment (start 115 142.5) (end 116.5 144) (width 0.2) (layer "F.Cu") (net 5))
 (segment (start 107.995 141.575) (end 108.92 142.5) (width 0.2) (layer "F.Cu") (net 5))
 (segment (start 150.007143 92.543744) (end 150.007143 109.742857) (width 0.2) (layer "F.Cu") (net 5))
 (segment (start 128.73 94.5) (end 130.686256 92.543744) (width 0.2) (layer "F.Cu") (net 5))
 (segment (start 116.5 144) (end 120.54 144) (width 0.2) (layer "F.Cu") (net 5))
 (segment (start 130.686256 92.543744) (end 150.007143 92.543744) (width 0.2) (layer "F.Cu") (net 5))
 (segment (start 108.92 142.5) (end 115 142.5) (width 0.2) (layer "F.Cu") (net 5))
 (segment (start 120.54 144) (end 120.72 144.18) (width 0.2) (layer "F.Cu") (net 5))
 (segment (start 150.007143 109.742857) (end 145.5 114.25) (width 0.2) (layer "F.Cu") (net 5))
 (segment (start 107.995 126.575) (end 109.5 125.07) (width 0.2) (layer "F.Cu") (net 7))
 (segment (start 109.5 125.07) (end 109.5 108.12) (width 0.2) (layer "F.Cu") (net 7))
 (segment (start 109.5 108.12) (end 119.16 98.46) (width 0.2) (layer "F.Cu") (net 7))
 (segment (start 119.16 98.46) (end 120.72 98.46) (width 0.2) (layer "F.Cu") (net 7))
 (segment (start 120.26 110.7) (end 120.72 111.16) (width 0.2) (layer "F.Cu") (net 11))
 (segment (start 108.925 136.575) (end 113.5 132) (width 0.2) (layer "F.Cu") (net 11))
 (segment (start 107.995 136.575) (end 108.925 136.575) (width 0.2) (layer "F.Cu") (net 11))
 (segment (start 113.5 116.82) (end 119.16 111.16) (width 0.2) (layer "F.Cu") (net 11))
 (segment (start 119.16 111.16) (end 120.72 111.16) (width 0.2) (layer "F.Cu") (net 11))
 (segment (start 113.5 132) (end 113.5 116.82) (width 0.2) (layer "F.Cu") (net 11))
 (segment (start 133.81 99.149709) (end 135.660291 101) (width 0.2) (layer "B.Cu") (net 26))
 (segment (start 135.660291 101) (end 138.5 101) (width 0.2) (layer "B.Cu") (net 26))
 (segment (start 133.81 94.5) (end 133.81 99.149709) (width 0.2) (layer "B.Cu") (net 26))
 (segment (start 126.19 94.5) (end 126.19 98.07) (width 0.2) (layer "F.Cu") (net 28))
 (segment (start 126.19 98.07) (end 120.72 103.54) (width 0.2) (layer "F.Cu") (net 28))
 (segment (start 131.27 94.5) (end 135.23 98.46) (width 0.2) (layer "F.Cu") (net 27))
 (segment (start 135.23 98.46) (end 138.5 98.46) (width 0.2) (layer "F.Cu") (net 27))
 (segment (start 138.66 111) (end 138.5 111.16) (width 0.2) (layer "F.Cu") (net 3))
 (segment (start 145.5 109.25) (end 143.963272 109.25) (width 0.2) (layer "B.Cu") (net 3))
 (segment (start 142.053272 111.16) (end 138.5 111.16) (width 0.2) (layer "B.Cu") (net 3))
 (segment (start 143.963272 109.25) (end 142.053272 111.16) (width 0.2) (layer "B.Cu") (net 3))
 (segment (start 138.7 113.5) (end 138.5 113.7) (width 0.2) (layer "F.Cu") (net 2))
 (segment (start 145.5 106.75) (end 147.524576 106.75) (width 0.2) (layer "B.Cu") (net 2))
 (segment (start 143.719818 118.5) (end 142.959626 117.739808) (width 0.2) (layer "B.Cu") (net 2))
 (segment (start 147.491767 118.5) (end 143.719818 118.5) (width 0.2) (layer "B.Cu") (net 2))
 (segment (start 148.274576 107.5) (end 148.274576 117.717191) (width 0.2) (layer "B.Cu") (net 2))
 (segment (start 142.959626 117.739808) (end 142.959626 114.844857) (width 0.2) (layer "B.Cu") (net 2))
 (segment (start 148.274576 117.717191) (end 147.491767 118.5) (width 0.2) (layer "B.Cu") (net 2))
 (segment (start 141.814769 113.7) (end 138.5 113.7) (width 0.2) (layer "B.Cu") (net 2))
 (segment (start 147.524576 106.75) (end 148.274576 107.5) (width 0.2) (layer "B.Cu") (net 2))
 (segment (start 142.959626 114.844857) (end 141.814769 113.7) (width 0.2) (layer "B.Cu") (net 2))
 (segment (start 138.62 108.5) (end 138.5 108.62) (width 0.2) (layer "F.Cu") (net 4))
 (segment (start 145.5 111.75) (end 142.37 108.62) (width 0.2) (layer "F.Cu") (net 4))
 (segment (start 142.37 108.62) (end 138.5 108.62) (width 0.2) (layer "F.Cu") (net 4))
 (segment (start 139.01 116.75) (end 138.5 116.24) (width 0.2) (layer "F.Cu") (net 6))
 (segment (start 145.5 116.75) (end 139.01 116.75) (width 0.2) (layer "F.Cu") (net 6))
 (segment (start 138.54 103.5) (end 138.5 103.54) (width 0.2) (layer "F.Cu") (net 25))
 (segment (start 143.67 106.08) (end 138.5 106.08) (width 0.2) (layer "F.Cu") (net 1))
 (segment (start 145.5 104.25) (end 143.67 106.08) (width 0.2) (layer "F.Cu") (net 1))
 (segment (start 120.5 119) (end 120.72 118.78) (width 0.2) (layer "B.Cu") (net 30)))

